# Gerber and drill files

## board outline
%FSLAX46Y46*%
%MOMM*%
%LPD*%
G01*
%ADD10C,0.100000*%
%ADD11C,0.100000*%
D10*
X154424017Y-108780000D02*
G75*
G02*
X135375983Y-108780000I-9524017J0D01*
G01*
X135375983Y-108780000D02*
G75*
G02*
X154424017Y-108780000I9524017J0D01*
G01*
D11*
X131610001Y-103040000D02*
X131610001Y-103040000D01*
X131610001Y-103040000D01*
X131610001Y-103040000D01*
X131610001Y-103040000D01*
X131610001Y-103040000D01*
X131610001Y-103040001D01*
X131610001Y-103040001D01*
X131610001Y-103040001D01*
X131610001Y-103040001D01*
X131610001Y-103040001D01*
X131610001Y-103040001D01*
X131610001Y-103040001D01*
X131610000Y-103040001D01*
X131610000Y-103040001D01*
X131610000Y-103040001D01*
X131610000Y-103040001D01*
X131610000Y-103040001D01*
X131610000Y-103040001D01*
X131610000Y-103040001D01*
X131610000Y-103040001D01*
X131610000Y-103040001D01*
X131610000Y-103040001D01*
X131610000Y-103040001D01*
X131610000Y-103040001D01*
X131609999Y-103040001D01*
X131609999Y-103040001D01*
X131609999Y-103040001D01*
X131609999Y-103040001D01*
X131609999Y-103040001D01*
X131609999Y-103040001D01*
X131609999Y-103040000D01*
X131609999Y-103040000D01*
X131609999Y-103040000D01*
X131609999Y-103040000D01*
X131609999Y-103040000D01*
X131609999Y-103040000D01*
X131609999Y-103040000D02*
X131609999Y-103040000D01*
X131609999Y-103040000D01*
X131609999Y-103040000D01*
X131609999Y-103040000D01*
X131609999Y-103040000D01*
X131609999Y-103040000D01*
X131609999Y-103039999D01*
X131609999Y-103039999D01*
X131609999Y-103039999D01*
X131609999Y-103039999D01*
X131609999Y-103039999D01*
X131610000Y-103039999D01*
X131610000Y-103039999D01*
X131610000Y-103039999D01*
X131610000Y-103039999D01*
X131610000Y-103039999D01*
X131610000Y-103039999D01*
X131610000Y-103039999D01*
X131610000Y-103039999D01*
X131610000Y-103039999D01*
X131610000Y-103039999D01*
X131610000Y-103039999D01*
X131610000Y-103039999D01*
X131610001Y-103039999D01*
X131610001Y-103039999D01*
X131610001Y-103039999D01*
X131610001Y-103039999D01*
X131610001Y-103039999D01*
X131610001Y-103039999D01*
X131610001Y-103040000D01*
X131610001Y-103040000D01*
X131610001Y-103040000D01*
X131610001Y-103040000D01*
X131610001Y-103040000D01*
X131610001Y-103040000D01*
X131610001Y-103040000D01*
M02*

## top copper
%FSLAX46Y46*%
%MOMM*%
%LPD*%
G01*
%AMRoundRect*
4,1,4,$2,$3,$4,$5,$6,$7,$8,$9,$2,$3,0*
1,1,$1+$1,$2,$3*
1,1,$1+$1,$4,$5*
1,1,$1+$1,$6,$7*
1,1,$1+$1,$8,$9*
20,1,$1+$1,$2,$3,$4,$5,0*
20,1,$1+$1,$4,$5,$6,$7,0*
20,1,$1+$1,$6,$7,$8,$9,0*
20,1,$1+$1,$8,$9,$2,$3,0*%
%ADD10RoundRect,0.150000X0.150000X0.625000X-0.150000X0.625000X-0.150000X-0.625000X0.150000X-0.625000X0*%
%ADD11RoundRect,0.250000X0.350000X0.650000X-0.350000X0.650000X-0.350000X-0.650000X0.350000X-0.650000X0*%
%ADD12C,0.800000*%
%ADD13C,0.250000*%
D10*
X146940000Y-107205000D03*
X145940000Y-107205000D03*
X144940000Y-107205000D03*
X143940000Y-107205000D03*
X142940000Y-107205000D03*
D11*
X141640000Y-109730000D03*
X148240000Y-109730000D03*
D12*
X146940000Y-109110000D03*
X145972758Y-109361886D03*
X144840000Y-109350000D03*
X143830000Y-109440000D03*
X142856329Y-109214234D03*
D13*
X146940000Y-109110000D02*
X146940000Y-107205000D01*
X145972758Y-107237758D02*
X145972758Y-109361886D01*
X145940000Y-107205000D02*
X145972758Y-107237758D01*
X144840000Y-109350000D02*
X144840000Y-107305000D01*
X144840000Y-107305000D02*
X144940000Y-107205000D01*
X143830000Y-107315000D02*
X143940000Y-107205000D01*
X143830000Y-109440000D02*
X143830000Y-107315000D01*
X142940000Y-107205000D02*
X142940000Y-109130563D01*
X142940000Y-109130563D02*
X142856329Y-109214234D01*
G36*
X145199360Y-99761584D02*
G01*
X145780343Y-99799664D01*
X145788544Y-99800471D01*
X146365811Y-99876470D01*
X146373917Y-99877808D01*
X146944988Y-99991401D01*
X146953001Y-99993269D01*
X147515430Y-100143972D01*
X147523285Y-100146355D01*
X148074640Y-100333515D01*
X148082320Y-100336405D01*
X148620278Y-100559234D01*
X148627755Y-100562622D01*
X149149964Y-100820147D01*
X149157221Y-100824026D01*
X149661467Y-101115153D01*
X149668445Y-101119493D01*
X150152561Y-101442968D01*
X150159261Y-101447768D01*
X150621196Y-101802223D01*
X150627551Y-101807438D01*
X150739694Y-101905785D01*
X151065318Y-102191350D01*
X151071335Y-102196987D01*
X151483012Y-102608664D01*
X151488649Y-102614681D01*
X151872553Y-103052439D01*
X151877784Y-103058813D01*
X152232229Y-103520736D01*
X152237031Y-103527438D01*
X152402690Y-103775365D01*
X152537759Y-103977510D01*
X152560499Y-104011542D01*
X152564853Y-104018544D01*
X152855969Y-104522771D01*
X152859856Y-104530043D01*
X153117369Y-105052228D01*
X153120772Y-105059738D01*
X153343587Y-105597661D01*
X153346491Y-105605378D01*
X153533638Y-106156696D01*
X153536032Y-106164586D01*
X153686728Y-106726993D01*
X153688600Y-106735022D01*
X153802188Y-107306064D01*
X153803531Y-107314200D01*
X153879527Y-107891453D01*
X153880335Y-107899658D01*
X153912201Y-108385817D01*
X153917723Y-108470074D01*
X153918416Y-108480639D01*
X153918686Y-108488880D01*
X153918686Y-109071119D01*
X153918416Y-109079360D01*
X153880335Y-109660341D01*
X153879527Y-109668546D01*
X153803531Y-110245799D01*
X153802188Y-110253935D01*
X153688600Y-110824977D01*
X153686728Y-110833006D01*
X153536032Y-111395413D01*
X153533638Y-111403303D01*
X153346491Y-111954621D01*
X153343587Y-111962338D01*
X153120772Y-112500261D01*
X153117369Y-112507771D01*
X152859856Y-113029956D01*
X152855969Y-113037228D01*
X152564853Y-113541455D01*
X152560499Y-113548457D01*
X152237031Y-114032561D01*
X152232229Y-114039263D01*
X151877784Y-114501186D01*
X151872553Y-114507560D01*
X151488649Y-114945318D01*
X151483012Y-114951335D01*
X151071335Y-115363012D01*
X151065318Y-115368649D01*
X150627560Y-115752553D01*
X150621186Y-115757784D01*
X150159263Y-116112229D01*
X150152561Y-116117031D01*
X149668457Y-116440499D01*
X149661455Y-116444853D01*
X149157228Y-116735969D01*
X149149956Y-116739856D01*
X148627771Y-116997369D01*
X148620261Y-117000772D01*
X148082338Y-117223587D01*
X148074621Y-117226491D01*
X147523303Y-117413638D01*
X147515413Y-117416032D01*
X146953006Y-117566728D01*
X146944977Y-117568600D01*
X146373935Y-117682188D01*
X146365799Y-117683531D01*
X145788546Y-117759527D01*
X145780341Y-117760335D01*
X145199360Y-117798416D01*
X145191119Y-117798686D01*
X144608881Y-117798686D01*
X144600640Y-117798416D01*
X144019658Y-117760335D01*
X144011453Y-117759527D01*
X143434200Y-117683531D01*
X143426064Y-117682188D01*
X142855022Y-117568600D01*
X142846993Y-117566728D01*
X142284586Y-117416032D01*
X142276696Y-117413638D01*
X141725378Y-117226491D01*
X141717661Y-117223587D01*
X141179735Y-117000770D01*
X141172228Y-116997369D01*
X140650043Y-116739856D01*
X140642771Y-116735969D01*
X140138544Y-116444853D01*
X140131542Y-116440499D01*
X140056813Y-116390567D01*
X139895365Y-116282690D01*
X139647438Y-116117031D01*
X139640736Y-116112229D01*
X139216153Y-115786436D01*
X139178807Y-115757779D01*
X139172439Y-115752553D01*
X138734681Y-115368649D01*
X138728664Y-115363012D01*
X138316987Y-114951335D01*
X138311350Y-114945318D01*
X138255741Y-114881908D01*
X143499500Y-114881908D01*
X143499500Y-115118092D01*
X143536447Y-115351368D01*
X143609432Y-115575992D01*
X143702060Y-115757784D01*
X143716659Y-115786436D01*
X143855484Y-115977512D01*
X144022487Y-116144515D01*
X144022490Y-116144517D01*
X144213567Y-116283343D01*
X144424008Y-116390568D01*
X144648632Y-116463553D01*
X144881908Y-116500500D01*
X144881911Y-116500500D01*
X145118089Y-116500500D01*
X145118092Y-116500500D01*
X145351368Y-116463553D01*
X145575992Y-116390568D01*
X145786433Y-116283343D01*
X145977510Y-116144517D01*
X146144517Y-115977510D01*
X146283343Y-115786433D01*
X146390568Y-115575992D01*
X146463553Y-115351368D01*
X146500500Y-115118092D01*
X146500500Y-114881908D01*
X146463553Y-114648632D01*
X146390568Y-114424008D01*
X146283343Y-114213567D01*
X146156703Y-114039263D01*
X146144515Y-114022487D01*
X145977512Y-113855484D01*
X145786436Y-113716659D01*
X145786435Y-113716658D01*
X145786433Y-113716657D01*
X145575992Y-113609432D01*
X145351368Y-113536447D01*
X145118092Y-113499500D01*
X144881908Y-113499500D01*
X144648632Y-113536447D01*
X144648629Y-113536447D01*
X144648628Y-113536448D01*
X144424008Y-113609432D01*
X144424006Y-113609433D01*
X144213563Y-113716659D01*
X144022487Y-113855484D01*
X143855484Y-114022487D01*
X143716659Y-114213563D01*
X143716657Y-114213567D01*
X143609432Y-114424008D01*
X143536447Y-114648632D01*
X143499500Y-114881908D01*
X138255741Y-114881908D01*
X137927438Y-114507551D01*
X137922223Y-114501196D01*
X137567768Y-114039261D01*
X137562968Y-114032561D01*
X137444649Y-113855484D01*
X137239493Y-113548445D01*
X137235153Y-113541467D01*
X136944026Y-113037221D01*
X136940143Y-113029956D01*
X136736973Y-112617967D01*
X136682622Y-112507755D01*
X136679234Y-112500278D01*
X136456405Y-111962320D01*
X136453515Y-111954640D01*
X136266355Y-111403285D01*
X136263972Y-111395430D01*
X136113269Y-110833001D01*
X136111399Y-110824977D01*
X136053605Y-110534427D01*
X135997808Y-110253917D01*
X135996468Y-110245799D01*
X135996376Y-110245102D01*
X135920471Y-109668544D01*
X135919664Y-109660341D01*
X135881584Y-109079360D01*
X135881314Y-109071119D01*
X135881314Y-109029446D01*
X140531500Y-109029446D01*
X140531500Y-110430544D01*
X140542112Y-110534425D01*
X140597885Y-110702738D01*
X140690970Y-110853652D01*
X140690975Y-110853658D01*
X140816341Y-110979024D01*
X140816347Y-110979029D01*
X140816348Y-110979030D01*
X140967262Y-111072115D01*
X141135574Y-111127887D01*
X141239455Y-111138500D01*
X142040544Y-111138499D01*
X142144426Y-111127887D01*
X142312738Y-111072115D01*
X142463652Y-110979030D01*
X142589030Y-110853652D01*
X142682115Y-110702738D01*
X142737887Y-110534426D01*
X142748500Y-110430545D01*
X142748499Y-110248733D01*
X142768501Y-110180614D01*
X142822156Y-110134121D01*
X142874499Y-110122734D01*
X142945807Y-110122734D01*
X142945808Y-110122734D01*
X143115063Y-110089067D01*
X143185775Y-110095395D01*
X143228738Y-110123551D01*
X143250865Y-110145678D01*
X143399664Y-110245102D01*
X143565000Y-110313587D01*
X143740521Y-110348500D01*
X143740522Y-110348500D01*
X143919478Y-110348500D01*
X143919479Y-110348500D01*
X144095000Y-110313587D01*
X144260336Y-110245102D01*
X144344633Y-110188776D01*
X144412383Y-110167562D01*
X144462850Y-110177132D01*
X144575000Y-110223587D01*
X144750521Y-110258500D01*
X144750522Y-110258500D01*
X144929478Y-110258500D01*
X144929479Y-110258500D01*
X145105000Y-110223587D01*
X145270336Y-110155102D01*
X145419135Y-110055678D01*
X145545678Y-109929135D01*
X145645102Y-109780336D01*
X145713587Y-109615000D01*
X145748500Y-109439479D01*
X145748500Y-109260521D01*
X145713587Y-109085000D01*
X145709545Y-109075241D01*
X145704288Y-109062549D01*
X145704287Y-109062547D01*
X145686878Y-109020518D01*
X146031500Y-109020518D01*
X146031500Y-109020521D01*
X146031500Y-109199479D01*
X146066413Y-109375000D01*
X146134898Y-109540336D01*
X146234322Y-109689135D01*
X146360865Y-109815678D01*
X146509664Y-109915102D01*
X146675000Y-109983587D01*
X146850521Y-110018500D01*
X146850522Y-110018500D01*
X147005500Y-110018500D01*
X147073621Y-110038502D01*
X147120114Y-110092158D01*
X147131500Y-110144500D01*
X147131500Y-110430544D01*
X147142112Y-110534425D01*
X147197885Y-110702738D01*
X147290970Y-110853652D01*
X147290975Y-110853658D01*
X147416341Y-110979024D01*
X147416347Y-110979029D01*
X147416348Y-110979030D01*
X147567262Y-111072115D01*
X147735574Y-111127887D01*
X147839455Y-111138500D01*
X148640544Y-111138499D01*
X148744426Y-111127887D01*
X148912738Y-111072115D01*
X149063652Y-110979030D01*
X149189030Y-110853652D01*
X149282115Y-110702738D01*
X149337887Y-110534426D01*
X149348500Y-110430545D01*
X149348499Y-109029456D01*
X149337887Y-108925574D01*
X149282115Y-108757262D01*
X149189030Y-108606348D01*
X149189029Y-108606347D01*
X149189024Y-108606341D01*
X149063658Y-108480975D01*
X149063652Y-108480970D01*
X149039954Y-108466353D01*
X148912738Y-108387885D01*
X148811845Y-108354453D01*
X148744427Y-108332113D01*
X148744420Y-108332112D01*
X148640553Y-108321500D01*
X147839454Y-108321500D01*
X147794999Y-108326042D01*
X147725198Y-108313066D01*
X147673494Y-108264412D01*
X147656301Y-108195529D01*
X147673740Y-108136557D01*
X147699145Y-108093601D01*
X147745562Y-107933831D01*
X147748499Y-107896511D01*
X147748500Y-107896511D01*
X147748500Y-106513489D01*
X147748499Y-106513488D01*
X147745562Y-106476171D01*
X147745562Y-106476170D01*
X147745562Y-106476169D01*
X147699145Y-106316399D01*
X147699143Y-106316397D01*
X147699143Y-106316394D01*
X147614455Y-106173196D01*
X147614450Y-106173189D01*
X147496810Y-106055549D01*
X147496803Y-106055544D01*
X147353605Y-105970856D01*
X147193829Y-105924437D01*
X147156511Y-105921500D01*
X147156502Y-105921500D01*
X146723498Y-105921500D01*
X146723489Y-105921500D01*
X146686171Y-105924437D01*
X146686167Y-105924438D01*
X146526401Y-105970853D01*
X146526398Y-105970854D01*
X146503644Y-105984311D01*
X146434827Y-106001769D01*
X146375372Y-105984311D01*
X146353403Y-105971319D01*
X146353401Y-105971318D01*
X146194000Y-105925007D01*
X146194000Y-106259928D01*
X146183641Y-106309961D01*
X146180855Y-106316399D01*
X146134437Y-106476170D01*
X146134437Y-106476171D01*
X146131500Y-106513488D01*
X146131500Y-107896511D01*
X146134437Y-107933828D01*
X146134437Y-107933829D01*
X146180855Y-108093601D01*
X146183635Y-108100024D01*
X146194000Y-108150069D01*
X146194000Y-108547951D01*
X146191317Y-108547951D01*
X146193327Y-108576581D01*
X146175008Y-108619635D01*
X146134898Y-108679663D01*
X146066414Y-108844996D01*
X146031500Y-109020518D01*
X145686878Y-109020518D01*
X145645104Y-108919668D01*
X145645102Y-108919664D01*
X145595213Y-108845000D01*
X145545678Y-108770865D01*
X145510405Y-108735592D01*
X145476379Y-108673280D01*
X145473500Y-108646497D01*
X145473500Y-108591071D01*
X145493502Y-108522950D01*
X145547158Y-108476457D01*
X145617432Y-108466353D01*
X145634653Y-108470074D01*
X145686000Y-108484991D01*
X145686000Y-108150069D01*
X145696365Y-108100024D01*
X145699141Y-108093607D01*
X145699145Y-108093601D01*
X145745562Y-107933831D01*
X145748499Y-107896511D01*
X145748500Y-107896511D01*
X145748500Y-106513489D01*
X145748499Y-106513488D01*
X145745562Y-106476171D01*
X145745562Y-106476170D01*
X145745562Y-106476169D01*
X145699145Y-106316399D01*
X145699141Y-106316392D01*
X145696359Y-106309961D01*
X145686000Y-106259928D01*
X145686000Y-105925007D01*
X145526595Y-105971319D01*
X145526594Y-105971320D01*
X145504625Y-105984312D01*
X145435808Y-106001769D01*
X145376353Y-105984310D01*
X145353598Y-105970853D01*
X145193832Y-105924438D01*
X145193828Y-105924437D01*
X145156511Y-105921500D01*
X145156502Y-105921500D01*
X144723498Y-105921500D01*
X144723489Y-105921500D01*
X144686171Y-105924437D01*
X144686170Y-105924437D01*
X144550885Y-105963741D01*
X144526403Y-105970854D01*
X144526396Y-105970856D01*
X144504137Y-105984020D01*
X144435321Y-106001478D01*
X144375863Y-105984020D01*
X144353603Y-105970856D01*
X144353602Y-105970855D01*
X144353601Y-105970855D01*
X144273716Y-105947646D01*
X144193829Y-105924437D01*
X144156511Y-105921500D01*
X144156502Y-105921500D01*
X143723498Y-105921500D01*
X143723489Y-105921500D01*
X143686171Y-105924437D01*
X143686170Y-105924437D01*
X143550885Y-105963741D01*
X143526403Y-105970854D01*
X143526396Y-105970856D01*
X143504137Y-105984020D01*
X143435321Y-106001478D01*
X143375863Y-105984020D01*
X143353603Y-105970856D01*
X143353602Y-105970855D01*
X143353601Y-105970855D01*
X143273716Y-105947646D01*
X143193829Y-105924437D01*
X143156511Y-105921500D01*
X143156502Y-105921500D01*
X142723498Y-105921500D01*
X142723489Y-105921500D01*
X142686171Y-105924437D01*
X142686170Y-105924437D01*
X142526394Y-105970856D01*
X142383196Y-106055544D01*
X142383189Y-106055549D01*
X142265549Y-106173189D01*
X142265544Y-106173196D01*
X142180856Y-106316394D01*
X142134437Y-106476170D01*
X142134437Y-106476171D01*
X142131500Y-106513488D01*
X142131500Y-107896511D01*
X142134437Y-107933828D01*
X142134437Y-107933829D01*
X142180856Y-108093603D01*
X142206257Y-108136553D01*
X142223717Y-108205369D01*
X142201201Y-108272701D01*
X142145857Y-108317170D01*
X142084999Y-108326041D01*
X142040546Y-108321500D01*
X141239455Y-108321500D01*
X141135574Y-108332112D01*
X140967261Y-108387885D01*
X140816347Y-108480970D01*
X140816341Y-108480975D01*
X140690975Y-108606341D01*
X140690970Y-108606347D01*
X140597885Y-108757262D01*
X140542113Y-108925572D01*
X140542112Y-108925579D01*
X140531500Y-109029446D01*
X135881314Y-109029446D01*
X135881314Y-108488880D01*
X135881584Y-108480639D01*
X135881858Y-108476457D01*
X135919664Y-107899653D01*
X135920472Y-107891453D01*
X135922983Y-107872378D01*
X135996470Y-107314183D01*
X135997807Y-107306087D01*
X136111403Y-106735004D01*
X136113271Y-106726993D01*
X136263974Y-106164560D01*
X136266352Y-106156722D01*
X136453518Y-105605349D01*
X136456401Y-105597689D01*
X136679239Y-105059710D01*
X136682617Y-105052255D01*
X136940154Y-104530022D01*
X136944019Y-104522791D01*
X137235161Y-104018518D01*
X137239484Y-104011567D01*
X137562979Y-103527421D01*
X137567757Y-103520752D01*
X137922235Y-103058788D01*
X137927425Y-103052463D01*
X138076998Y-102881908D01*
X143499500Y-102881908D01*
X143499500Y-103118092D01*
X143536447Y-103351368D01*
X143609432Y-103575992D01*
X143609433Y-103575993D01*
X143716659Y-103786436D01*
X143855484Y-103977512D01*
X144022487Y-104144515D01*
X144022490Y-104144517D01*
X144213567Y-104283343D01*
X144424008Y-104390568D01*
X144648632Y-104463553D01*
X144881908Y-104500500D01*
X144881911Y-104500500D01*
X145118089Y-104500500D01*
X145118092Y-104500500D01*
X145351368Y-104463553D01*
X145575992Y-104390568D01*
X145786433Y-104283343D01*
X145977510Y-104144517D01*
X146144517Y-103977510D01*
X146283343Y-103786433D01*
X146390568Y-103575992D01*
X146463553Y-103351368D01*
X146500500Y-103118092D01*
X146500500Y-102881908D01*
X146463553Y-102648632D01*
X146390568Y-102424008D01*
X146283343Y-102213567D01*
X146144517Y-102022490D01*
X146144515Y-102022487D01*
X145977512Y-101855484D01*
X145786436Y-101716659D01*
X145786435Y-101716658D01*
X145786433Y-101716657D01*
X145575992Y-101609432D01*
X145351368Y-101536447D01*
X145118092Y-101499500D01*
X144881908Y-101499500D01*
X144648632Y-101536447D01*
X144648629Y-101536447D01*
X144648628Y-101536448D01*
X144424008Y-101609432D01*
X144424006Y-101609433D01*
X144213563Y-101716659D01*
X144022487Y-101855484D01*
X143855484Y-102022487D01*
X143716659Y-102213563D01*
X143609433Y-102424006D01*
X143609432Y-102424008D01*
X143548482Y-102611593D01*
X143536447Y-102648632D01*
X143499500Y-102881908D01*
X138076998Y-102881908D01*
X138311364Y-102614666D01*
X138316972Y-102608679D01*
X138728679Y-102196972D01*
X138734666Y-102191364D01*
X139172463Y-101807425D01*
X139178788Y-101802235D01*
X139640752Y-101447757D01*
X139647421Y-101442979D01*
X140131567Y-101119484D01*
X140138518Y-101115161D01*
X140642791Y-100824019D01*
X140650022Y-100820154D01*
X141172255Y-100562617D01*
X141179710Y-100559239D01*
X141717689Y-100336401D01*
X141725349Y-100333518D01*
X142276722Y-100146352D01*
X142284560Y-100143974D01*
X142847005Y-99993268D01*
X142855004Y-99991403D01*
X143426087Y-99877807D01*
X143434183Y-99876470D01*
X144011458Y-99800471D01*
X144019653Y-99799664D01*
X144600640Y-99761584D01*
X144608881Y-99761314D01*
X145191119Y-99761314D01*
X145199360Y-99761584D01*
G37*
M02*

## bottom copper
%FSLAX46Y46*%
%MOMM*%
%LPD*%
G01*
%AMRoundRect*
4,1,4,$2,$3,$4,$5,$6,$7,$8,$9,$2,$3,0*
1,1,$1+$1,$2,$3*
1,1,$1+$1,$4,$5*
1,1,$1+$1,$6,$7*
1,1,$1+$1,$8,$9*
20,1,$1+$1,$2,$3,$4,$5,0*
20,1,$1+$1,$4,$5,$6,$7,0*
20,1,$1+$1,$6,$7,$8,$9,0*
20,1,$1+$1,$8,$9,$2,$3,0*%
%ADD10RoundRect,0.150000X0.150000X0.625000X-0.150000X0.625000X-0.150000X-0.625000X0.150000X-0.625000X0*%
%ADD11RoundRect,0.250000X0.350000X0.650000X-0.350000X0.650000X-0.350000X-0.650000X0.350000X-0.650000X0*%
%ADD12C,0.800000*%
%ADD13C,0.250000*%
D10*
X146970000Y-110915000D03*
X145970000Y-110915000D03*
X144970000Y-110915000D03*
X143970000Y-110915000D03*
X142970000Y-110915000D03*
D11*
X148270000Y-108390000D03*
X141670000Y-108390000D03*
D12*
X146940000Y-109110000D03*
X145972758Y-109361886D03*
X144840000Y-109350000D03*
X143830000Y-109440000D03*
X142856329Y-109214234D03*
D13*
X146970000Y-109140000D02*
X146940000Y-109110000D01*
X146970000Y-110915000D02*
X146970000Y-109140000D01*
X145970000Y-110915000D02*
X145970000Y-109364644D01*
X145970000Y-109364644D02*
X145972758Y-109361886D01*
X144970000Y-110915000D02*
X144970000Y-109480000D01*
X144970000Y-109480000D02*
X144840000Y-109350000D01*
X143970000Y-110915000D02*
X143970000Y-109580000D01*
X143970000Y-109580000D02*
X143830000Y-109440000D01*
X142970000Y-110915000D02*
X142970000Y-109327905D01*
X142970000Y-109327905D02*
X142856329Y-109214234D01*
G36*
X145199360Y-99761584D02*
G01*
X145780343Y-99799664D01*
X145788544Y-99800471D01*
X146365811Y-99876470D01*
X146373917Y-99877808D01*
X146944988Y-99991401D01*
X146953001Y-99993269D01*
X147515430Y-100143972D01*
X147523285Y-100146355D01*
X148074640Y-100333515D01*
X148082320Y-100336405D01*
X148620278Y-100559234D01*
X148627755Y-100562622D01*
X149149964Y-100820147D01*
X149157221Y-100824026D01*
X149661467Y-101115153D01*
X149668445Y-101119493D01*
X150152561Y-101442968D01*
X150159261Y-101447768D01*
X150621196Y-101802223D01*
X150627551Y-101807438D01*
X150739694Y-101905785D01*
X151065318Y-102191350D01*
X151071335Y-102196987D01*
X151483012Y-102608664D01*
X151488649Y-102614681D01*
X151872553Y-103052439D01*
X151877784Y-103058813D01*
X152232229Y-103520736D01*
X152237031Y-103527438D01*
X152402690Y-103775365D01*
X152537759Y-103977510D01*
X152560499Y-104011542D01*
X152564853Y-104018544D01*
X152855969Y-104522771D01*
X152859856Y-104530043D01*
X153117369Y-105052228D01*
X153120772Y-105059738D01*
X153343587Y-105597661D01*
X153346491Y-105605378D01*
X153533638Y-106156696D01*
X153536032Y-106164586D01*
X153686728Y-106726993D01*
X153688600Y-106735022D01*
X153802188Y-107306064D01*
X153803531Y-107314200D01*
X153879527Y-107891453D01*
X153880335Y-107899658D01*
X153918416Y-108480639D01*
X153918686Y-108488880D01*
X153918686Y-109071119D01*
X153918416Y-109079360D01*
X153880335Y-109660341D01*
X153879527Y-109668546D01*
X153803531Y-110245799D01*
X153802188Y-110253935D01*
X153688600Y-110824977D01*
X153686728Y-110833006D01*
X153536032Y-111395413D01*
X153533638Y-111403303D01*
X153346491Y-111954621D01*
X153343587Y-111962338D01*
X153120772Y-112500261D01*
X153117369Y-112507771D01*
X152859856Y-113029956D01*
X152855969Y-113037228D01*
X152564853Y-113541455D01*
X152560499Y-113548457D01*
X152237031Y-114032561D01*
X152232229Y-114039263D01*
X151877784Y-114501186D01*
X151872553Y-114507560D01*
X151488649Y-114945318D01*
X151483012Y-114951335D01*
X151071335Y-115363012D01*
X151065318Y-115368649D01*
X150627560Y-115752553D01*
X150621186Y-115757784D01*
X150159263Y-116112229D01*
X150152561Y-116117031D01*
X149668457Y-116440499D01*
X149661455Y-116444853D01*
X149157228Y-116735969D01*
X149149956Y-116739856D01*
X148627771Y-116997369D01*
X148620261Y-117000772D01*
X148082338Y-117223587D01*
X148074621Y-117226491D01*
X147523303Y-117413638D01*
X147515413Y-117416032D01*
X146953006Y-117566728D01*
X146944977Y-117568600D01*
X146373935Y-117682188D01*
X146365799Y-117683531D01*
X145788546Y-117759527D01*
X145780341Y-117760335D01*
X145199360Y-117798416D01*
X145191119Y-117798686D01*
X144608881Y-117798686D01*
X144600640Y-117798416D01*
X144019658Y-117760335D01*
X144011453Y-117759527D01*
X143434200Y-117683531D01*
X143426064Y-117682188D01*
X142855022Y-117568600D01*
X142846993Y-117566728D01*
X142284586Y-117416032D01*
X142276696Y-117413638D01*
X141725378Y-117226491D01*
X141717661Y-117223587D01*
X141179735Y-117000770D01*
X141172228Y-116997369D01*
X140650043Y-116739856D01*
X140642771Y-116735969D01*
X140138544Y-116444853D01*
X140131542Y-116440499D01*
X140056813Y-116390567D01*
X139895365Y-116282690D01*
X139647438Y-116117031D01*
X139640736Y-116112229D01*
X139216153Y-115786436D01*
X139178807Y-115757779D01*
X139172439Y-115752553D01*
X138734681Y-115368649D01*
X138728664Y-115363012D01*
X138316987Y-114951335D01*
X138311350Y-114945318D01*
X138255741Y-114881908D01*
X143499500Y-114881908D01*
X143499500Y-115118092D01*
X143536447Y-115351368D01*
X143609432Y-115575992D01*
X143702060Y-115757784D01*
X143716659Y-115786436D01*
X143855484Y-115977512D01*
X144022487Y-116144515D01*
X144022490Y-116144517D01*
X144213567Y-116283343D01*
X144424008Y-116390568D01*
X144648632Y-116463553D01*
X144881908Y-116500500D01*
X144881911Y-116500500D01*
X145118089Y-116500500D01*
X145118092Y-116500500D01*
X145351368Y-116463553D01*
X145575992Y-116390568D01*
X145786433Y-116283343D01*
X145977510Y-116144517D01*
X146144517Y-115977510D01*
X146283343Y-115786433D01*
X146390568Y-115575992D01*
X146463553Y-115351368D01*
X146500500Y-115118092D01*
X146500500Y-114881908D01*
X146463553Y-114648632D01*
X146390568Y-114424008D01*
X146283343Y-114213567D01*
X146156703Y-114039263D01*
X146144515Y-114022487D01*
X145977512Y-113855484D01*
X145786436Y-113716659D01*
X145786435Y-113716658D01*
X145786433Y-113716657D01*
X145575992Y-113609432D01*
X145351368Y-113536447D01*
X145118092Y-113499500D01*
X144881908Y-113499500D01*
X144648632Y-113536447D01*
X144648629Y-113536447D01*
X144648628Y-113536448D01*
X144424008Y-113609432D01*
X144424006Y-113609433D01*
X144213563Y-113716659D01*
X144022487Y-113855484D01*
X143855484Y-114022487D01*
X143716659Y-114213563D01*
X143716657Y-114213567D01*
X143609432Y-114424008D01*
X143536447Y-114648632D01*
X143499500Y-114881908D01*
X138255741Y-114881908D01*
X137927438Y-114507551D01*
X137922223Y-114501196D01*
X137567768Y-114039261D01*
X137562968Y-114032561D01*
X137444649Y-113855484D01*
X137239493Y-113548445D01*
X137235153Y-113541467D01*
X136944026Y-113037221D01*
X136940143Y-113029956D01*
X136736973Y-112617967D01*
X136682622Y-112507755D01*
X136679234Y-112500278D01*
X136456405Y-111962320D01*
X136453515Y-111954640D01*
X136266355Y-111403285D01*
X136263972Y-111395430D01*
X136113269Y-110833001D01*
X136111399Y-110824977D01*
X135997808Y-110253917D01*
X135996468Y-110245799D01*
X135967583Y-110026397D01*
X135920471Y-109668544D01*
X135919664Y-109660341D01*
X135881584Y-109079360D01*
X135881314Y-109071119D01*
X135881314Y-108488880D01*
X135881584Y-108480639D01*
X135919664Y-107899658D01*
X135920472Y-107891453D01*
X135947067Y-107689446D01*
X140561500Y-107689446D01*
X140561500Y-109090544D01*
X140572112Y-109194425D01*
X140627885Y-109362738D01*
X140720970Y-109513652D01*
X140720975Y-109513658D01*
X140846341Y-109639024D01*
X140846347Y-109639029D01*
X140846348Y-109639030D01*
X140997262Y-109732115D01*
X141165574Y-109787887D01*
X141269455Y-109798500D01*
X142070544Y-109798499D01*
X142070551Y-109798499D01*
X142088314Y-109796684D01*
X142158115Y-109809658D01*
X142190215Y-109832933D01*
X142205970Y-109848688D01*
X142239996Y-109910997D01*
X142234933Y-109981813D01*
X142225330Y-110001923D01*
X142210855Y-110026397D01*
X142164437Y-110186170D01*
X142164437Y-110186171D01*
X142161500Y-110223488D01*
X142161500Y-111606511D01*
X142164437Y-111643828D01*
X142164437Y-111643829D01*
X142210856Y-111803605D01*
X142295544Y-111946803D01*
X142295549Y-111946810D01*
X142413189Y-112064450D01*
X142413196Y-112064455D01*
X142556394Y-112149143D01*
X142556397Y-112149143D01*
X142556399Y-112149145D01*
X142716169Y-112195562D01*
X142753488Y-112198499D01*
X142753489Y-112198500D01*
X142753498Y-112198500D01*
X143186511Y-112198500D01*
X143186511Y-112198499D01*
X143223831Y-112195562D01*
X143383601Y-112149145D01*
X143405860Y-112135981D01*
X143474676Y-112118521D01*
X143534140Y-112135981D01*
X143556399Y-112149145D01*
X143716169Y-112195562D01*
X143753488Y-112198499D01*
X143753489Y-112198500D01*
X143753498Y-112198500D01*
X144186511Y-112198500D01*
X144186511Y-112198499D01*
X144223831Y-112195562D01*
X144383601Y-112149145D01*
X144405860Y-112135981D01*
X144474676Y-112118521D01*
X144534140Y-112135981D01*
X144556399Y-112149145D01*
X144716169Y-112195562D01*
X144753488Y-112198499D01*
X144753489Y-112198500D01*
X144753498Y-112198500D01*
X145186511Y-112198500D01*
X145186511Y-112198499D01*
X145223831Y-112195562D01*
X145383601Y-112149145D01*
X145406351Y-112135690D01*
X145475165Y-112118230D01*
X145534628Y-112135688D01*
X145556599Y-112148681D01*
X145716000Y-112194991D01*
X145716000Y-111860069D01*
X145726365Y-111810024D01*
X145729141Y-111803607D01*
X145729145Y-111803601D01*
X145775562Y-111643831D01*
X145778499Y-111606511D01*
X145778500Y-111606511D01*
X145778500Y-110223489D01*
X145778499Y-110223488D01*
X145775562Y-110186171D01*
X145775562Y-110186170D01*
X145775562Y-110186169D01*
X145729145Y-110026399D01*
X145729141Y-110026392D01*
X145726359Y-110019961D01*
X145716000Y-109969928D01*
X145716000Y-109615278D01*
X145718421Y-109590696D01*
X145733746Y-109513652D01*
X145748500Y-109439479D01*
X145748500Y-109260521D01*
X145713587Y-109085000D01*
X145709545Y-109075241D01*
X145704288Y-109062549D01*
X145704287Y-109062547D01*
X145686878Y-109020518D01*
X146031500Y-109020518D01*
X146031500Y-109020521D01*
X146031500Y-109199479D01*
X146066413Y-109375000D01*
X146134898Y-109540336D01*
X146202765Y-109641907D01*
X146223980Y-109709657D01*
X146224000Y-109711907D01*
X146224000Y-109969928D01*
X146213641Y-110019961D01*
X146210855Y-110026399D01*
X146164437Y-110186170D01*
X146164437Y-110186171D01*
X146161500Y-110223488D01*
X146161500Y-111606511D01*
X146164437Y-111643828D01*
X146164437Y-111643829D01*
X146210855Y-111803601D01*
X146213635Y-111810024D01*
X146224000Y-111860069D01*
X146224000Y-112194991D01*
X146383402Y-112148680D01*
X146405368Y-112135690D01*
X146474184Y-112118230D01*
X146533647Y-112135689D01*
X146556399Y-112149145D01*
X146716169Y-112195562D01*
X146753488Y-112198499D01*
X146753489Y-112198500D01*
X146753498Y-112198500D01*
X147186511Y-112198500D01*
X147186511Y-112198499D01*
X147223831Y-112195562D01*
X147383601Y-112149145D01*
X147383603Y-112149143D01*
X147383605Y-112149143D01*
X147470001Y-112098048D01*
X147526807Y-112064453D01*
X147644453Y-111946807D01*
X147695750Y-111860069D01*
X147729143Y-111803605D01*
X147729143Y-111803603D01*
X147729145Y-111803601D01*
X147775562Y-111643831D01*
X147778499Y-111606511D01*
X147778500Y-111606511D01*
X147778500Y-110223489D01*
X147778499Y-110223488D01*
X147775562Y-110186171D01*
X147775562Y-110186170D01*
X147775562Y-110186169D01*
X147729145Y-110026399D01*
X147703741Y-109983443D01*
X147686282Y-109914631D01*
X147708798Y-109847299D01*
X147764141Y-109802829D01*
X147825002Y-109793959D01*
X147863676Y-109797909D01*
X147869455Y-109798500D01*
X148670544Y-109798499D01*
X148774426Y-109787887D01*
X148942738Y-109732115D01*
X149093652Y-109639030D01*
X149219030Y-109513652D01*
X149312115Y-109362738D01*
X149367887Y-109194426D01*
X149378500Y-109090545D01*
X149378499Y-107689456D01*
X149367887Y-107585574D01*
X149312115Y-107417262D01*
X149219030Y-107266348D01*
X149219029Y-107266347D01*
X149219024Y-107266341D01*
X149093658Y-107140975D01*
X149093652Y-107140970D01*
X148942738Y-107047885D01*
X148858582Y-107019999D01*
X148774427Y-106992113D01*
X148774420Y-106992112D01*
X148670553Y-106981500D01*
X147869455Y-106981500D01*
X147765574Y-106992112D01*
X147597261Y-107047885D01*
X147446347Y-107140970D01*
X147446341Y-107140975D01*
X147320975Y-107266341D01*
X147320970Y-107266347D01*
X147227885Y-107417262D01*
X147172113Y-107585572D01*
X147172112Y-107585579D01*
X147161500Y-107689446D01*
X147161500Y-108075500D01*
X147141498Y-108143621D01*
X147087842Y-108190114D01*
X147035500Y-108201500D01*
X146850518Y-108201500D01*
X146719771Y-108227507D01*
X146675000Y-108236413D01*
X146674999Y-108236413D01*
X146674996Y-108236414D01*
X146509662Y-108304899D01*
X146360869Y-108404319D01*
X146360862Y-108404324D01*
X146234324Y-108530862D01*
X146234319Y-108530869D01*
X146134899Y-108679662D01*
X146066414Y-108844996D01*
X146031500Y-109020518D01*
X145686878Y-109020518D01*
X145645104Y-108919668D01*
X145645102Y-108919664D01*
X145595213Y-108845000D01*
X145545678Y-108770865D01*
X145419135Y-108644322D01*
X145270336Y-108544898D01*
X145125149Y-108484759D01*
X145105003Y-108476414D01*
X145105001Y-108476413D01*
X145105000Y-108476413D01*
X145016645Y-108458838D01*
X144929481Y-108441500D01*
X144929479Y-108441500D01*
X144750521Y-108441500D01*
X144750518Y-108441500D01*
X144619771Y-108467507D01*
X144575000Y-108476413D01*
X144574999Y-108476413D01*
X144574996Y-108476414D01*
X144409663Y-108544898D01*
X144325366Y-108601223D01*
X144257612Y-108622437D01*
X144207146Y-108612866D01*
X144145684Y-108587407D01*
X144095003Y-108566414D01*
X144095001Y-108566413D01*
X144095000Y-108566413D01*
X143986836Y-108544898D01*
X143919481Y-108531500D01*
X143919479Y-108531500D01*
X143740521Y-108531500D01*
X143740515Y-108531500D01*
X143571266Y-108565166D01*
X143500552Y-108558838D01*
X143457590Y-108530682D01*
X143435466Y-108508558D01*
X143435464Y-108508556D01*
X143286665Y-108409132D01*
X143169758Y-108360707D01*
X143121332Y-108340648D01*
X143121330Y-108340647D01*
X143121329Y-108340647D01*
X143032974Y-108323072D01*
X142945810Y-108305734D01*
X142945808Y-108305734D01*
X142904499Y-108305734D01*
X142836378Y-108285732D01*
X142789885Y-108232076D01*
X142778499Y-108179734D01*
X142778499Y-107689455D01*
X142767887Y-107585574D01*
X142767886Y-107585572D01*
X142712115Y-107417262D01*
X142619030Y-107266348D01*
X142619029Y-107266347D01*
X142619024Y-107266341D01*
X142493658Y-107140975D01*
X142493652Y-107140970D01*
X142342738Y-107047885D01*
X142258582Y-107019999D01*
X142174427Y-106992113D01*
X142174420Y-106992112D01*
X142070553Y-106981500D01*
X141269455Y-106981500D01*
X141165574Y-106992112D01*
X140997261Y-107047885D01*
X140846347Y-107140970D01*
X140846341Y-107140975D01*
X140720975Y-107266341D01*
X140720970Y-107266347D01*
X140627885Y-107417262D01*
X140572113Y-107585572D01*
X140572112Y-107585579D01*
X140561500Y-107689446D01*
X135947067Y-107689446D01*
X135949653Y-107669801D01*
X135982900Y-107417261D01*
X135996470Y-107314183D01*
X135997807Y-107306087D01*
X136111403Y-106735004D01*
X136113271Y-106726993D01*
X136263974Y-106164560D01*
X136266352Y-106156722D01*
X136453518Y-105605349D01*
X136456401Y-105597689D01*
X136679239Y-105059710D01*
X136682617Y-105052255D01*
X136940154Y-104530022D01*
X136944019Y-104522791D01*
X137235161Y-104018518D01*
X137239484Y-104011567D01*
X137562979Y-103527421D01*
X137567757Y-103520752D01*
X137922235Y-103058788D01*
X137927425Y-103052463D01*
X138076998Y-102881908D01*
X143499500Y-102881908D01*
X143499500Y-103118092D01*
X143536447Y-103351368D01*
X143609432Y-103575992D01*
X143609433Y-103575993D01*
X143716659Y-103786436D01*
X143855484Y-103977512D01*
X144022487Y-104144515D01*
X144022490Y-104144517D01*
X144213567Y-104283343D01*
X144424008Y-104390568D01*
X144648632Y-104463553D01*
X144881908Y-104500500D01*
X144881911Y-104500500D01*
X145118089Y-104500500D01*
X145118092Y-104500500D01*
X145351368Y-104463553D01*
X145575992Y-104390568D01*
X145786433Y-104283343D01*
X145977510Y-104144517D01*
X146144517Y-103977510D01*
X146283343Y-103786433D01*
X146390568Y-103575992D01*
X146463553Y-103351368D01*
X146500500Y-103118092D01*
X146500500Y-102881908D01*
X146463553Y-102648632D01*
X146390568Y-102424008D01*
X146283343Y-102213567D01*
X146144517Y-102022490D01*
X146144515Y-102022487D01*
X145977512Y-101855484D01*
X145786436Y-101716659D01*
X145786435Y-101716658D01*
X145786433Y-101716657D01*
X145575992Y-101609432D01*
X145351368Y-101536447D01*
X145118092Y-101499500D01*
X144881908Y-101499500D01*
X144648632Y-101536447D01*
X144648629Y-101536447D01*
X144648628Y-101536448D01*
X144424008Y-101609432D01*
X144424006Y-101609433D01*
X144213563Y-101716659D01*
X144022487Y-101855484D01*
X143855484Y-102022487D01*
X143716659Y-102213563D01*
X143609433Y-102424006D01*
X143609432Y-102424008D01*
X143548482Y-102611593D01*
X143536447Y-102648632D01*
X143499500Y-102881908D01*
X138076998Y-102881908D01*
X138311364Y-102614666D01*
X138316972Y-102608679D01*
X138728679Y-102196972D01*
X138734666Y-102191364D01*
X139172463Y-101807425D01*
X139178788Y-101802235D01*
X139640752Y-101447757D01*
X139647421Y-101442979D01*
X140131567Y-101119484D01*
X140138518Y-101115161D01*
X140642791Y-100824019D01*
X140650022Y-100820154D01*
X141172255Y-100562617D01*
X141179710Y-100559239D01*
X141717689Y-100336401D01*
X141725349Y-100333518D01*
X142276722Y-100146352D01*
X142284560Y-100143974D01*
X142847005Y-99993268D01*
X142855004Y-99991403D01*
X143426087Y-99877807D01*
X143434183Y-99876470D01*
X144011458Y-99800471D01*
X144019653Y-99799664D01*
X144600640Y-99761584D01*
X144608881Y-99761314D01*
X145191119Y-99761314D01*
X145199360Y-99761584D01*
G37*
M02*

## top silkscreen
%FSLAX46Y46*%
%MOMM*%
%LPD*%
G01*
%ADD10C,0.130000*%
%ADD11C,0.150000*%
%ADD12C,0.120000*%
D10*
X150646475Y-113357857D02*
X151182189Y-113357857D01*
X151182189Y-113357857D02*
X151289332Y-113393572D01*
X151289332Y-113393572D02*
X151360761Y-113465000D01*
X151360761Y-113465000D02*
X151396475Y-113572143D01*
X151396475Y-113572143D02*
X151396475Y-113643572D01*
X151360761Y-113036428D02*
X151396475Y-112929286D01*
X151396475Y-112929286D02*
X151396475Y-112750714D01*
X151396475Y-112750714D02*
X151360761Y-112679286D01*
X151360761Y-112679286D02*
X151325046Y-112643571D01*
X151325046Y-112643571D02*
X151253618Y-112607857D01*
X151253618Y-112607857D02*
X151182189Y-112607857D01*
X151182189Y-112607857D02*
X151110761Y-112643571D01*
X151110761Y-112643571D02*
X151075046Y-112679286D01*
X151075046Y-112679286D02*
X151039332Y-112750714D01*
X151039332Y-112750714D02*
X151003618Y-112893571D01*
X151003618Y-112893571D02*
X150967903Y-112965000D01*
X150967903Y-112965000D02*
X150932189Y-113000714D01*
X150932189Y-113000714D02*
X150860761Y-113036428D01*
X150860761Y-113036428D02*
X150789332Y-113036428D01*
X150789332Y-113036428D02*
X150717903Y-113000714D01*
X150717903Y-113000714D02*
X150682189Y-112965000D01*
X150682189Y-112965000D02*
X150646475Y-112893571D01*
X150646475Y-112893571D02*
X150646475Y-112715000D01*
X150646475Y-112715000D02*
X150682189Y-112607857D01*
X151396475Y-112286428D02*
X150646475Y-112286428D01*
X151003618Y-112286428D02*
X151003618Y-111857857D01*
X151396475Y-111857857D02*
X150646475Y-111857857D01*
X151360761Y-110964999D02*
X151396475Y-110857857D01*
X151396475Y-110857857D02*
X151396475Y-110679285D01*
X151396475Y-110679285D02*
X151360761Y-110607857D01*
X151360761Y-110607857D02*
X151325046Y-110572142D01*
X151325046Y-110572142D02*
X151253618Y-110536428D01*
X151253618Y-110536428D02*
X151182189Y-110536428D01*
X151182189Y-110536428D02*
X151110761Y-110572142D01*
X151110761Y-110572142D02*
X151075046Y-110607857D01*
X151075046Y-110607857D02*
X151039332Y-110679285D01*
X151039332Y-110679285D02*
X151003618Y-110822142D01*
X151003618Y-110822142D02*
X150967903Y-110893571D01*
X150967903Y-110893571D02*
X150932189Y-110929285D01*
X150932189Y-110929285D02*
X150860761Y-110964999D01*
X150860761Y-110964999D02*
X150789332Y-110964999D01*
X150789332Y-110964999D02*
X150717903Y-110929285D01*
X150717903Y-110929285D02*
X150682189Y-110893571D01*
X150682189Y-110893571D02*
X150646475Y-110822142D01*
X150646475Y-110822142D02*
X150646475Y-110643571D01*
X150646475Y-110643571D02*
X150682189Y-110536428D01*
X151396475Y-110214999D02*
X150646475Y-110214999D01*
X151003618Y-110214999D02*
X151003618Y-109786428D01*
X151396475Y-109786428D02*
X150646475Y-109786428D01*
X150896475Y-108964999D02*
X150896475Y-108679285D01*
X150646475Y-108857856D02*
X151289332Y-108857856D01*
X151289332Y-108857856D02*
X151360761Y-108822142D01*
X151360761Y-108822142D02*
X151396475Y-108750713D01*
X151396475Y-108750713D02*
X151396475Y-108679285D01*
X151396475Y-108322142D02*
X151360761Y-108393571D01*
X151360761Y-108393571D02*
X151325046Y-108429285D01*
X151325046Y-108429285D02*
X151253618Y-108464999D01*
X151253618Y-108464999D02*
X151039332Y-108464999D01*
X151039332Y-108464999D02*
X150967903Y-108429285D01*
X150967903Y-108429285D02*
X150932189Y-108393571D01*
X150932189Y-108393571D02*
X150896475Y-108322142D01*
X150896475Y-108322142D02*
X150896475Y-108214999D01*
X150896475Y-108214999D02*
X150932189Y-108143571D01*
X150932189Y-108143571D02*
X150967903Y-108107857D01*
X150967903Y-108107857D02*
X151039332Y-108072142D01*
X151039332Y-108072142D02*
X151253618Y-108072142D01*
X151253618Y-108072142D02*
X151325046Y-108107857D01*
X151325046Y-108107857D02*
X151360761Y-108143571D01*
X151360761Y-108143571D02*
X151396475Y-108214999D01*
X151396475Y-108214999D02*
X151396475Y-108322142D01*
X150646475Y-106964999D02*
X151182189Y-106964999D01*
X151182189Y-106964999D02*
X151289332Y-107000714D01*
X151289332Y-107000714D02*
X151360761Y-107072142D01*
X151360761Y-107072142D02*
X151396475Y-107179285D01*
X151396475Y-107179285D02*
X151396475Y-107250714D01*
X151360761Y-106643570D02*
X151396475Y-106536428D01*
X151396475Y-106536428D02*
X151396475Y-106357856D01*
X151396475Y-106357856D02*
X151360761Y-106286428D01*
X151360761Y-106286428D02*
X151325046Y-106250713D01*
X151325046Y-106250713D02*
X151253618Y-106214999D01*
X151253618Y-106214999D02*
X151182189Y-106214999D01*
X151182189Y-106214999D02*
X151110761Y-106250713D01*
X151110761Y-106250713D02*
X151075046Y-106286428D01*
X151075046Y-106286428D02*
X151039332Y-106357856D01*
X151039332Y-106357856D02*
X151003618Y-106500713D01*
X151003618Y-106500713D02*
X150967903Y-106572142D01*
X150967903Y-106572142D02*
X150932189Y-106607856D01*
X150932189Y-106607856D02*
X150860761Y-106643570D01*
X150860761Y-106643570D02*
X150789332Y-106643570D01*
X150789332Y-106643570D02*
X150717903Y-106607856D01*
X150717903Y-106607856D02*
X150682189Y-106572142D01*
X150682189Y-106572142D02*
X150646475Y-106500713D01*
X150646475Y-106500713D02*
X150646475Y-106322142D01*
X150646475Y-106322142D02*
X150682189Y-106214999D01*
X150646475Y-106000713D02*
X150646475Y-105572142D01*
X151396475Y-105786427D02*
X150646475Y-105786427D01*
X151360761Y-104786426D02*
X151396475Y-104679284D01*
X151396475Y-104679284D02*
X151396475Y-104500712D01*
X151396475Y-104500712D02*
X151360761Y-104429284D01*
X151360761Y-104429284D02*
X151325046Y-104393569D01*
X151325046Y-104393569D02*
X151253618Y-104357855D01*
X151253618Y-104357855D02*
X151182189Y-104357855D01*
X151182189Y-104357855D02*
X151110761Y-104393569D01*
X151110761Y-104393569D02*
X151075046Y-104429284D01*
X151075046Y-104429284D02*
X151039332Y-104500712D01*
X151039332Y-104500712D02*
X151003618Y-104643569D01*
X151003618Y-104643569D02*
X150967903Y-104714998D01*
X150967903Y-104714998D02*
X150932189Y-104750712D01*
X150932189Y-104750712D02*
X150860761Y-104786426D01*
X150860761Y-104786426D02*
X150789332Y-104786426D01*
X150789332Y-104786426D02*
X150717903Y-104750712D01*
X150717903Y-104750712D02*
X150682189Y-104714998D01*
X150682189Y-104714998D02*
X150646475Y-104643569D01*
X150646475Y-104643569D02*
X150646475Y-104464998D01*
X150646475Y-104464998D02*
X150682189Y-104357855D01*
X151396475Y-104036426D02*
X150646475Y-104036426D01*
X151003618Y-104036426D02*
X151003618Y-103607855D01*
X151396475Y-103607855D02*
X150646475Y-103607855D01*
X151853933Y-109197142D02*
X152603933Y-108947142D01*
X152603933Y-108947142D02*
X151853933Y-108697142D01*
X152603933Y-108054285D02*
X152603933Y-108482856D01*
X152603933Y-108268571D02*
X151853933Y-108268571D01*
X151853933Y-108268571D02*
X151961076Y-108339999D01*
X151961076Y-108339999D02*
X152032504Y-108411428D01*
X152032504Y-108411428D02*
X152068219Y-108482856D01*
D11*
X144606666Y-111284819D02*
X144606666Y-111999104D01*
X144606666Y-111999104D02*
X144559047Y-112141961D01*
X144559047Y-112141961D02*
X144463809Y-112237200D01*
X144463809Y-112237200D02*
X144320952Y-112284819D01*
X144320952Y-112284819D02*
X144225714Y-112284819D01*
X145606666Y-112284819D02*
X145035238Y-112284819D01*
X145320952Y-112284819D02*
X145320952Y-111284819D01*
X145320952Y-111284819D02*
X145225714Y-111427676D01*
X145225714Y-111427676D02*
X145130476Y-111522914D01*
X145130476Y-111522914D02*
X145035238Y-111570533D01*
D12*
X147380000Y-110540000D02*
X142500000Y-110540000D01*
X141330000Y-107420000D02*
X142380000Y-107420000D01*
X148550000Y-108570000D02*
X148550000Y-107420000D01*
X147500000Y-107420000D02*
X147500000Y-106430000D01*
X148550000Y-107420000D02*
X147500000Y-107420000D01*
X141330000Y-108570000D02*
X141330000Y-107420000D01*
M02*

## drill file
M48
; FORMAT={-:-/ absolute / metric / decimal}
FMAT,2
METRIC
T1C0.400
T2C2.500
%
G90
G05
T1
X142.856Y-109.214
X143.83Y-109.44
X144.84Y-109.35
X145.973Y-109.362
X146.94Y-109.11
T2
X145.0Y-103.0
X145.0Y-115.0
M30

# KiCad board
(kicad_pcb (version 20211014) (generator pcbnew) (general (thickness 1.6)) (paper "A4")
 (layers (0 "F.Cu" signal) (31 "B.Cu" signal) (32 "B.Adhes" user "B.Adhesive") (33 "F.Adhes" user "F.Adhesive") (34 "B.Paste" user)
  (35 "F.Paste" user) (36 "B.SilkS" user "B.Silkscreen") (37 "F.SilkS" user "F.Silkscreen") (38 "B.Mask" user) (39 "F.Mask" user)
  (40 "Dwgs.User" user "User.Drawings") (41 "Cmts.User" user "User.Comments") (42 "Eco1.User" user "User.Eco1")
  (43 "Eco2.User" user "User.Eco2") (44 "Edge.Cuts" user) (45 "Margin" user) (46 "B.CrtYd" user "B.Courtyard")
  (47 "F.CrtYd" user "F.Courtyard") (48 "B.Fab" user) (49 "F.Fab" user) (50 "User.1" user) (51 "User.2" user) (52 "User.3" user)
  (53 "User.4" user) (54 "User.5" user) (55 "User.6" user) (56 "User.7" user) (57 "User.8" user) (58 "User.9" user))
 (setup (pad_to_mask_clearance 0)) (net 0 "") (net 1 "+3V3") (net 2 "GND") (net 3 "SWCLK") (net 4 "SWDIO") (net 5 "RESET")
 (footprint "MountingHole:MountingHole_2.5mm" (layer "F.Cu") (at 145 103)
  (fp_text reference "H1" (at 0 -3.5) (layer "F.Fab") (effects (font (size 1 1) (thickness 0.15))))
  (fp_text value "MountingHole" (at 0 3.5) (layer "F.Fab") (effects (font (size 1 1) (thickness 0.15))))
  (pad "" np_thru_hole circle locked (at 0 0) (size 2.5 2.5) (drill 2.5) (layers *.Cu *.Mask)))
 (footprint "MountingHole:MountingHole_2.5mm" (layer "F.Cu") (at 145 115)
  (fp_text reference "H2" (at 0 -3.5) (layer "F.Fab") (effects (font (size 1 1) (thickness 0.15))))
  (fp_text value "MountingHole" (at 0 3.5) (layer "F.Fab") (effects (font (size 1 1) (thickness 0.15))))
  (pad "" np_thru_hole circle locked (at 0 0) (size 2.5 2.5) (drill 2.5) (layers *.Cu *.Mask)))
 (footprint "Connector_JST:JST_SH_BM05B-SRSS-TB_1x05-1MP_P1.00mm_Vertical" (layer "F.Cu") (at 144.94 108.53 180)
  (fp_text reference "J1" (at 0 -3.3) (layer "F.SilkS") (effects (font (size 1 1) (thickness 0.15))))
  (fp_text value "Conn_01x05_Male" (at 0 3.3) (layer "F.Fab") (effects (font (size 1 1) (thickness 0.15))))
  (fp_line (start -2.44 -2.01) (end 2.44 -2.01) (layer "F.SilkS") (width 0.12))
  (fp_line (start 3.61 1.11) (end 2.56 1.11) (layer "F.SilkS") (width 0.12))
  (fp_line (start -3.61 -0.04) (end -3.61 1.11) (layer "F.SilkS") (width 0.12))
  (fp_line (start -2.56 1.11) (end -2.56 2.1) (layer "F.SilkS") (width 0.12))
  (fp_line (start -3.61 1.11) (end -2.56 1.11) (layer "F.SilkS") (width 0.12))
  (fp_line (start 3.61 -0.04) (end 3.61 1.11) (layer "F.SilkS") (width 0.12))
  (pad "1" smd roundrect locked (at -2 1.325 180) (size 0.6 1.55) (layers "F.Cu" "F.Paste" "F.Mask") (roundrect_rratio 0.25) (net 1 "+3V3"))
  (pad "2" smd roundrect locked (at -1 1.325 180) (size 0.6 1.55) (layers "F.Cu" "F.Paste" "F.Mask") (roundrect_rratio 0.25) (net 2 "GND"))
  (pad "3" smd roundrect locked (at 0 1.325 180) (size 0.6 1.55) (layers "F.Cu" "F.Paste" "F.Mask") (roundrect_rratio 0.25) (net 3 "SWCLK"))
  (pad "4" smd roundrect locked (at 1 1.325 180) (size 0.6 1.55) (layers "F.Cu" "F.Paste" "F.Mask") (roundrect_rratio 0.25) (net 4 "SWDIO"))
  (pad "5" smd roundrect locked (at 2 1.325 180) (size 0.6 1.55) (layers "F.Cu" "F.Paste" "F.Mask") (roundrect_rratio 0.25) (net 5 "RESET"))
  (pad "MP" smd roundrect locked (at 3.3 -1.2 180) (size 1.2 1.8) (layers "F.Cu" "F.Paste" "F.Mask") (roundrect_rratio 0.2083333333))
  (pad "MP" smd roundrect locked (at -3.3 -1.2 180) (size 1.2 1.8) (layers "F.Cu" "F.Paste" "F.Mask") (roundrect_rratio 0.2083333333)))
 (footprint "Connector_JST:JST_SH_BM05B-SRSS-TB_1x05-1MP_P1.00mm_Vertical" (layer "B.Cu") (at 144.97 109.59 180)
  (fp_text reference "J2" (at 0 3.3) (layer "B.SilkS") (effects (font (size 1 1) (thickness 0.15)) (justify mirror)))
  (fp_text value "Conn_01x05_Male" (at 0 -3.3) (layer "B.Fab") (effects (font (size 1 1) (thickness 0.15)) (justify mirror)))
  (pad "1" smd roundrect locked (at -2 -1.325 180) (size 0.6 1.55) (layers "B.Cu" "B.Paste" "B.Mask") (roundrect_rratio 0.25) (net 1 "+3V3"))
  (pad "2" smd roundrect locked (at -1 -1.325 180) (size 0.6 1.55) (layers "B.Cu" "B.Paste" "B.Mask") (roundrect_rratio 0.25) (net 2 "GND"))
  (pad "3" smd roundrect locked (at 0 -1.325 180) (size 0.6 1.55) (layers "B.Cu" "B.Paste" "B.Mask") (roundrect_rratio 0.25) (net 3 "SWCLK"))
  (pad "4" smd roundrect locked (at 1 -1.325 180) (size 0.6 1.55) (layers "B.Cu" "B.Paste" "B.Mask") (roundrect_rratio 0.25) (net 4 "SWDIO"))
  (pad "5" smd roundrect locked (at 2 -1.325 180) (size 0.6 1.55) (layers "B.Cu" "B.Paste" "B.Mask") (roundrect_rratio 0.25) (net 5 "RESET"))
  (pad "MP" smd roundrect locked (at -3.3 1.2 180) (size 1.2 1.8) (layers "B.Cu" "B.Paste" "B.Mask") (roundrect_rratio 0.2083333333))
  (pad "MP" smd roundrect locked (at 3.3 1.2 180) (size 1.2 1.8) (layers "B.Cu" "B.Paste" "B.Mask") (roundrect_rratio 0.2083333333)))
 (gr_circle (center 144.9 108.78) (end 153.52 112.83) (layer "Edge.Cuts") (width 0.1) (fill none))
 (gr_circle (center 131.61 103.04) (end 131.61 103.04) (layer "Edge.Cuts") (width 0.1) (fill none))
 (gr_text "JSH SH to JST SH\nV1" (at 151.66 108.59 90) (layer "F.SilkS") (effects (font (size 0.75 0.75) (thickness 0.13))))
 (segment (start 146.94 109.11) (end 146.94 107.205) (width 0.25) (layer "F.Cu") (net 1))
 (via (at 146.94 109.11) (size 0.8) (drill 0.4) (layers "F.Cu" "B.Cu") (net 1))
 (segment (start 146.97 109.14) (end 146.94 109.11) (width 0.25) (layer "B.Cu") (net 1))
 (segment (start 146.97 110.915) (end 146.97 109.14) (width 0.25) (layer "B.Cu") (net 1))
 (segment (start 145.972758 107.237758) (end 145.972758 109.361886) (width 0.25) (layer "F.Cu") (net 2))
 (segment (start 145.94 107.205) (end 145.972758 107.237758) (width 0.25) (layer "F.Cu") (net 2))
 (via (at 145.972758 109.361886) (size 0.8) (drill 0.4) (layers "F.Cu" "B.Cu") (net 2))
 (segment (start 145.97 110.915) (end 145.97 109.364644) (width 0.25) (layer "B.Cu") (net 2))
 (segment (start 145.97 109.364644) (end 145.972758 109.361886) (width 0.25) (layer "B.Cu") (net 2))
 (segment (start 144.84 109.35) (end 144.84 107.305) (width 0.25) (layer "F.Cu") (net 3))
 (segment (start 144.84 107.305) (end 144.94 107.205) (width 0.25) (layer "F.Cu") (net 3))
 (via (at 144.84 109.35) (size 0.8) (drill 0.4) (layers "F.Cu" "B.Cu") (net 3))
 (segment (start 144.97 110.915) (end 144.97 109.48) (width 0.25) (layer "B.Cu") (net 3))
 (segment (start 144.97 109.48) (end 144.84 109.35) (width 0.25) (layer "B.Cu") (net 3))
 (segment (start 143.83 107.315) (end 143.94 107.205) (width 0.25) (layer "F.Cu") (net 4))
 (segment (start 143.83 109.44) (end 143.83 107.315) (width 0.25) (layer "F.Cu") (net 4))
 (via (at 143.83 109.44) (size 0.8) (drill 0.4) (layers "F.Cu" "B.Cu") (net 4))
 (segment (start 143.97 110.915) (end 143.97 109.58) (width 0.25) (layer "B.Cu") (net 4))
 (segment (start 143.97 109.58) (end 143.83 109.44) (width 0.25) (layer "B.Cu") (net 4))
 (segment (start 142.94 107.205) (end 142.94 109.130563) (width 0.25) (layer "F.Cu") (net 5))
 (segment (start 142.94 109.130563) (end 142.856329 109.214234) (width 0.25) (layer "F.Cu") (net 5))
 (via (at 142.856329 109.214234) (size 0.8) (drill 0.4) (layers "F.Cu" "B.Cu") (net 5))
 (segment (start 142.97 110.915) (end 142.97 109.327905) (width 0.25) (layer "B.Cu") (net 5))
 (segment (start 142.97 109.327905) (end 142.856329 109.214234) (width 0.25) (layer "B.Cu") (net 5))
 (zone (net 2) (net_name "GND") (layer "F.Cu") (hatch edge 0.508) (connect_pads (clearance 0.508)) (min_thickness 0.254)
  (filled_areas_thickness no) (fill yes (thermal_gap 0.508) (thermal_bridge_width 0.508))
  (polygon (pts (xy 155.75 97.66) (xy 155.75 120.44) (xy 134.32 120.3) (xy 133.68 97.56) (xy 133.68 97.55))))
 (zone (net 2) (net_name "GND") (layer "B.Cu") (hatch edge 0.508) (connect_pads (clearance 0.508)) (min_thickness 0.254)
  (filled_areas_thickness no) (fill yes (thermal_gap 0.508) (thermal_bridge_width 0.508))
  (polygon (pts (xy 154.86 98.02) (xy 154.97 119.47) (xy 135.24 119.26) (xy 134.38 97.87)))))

